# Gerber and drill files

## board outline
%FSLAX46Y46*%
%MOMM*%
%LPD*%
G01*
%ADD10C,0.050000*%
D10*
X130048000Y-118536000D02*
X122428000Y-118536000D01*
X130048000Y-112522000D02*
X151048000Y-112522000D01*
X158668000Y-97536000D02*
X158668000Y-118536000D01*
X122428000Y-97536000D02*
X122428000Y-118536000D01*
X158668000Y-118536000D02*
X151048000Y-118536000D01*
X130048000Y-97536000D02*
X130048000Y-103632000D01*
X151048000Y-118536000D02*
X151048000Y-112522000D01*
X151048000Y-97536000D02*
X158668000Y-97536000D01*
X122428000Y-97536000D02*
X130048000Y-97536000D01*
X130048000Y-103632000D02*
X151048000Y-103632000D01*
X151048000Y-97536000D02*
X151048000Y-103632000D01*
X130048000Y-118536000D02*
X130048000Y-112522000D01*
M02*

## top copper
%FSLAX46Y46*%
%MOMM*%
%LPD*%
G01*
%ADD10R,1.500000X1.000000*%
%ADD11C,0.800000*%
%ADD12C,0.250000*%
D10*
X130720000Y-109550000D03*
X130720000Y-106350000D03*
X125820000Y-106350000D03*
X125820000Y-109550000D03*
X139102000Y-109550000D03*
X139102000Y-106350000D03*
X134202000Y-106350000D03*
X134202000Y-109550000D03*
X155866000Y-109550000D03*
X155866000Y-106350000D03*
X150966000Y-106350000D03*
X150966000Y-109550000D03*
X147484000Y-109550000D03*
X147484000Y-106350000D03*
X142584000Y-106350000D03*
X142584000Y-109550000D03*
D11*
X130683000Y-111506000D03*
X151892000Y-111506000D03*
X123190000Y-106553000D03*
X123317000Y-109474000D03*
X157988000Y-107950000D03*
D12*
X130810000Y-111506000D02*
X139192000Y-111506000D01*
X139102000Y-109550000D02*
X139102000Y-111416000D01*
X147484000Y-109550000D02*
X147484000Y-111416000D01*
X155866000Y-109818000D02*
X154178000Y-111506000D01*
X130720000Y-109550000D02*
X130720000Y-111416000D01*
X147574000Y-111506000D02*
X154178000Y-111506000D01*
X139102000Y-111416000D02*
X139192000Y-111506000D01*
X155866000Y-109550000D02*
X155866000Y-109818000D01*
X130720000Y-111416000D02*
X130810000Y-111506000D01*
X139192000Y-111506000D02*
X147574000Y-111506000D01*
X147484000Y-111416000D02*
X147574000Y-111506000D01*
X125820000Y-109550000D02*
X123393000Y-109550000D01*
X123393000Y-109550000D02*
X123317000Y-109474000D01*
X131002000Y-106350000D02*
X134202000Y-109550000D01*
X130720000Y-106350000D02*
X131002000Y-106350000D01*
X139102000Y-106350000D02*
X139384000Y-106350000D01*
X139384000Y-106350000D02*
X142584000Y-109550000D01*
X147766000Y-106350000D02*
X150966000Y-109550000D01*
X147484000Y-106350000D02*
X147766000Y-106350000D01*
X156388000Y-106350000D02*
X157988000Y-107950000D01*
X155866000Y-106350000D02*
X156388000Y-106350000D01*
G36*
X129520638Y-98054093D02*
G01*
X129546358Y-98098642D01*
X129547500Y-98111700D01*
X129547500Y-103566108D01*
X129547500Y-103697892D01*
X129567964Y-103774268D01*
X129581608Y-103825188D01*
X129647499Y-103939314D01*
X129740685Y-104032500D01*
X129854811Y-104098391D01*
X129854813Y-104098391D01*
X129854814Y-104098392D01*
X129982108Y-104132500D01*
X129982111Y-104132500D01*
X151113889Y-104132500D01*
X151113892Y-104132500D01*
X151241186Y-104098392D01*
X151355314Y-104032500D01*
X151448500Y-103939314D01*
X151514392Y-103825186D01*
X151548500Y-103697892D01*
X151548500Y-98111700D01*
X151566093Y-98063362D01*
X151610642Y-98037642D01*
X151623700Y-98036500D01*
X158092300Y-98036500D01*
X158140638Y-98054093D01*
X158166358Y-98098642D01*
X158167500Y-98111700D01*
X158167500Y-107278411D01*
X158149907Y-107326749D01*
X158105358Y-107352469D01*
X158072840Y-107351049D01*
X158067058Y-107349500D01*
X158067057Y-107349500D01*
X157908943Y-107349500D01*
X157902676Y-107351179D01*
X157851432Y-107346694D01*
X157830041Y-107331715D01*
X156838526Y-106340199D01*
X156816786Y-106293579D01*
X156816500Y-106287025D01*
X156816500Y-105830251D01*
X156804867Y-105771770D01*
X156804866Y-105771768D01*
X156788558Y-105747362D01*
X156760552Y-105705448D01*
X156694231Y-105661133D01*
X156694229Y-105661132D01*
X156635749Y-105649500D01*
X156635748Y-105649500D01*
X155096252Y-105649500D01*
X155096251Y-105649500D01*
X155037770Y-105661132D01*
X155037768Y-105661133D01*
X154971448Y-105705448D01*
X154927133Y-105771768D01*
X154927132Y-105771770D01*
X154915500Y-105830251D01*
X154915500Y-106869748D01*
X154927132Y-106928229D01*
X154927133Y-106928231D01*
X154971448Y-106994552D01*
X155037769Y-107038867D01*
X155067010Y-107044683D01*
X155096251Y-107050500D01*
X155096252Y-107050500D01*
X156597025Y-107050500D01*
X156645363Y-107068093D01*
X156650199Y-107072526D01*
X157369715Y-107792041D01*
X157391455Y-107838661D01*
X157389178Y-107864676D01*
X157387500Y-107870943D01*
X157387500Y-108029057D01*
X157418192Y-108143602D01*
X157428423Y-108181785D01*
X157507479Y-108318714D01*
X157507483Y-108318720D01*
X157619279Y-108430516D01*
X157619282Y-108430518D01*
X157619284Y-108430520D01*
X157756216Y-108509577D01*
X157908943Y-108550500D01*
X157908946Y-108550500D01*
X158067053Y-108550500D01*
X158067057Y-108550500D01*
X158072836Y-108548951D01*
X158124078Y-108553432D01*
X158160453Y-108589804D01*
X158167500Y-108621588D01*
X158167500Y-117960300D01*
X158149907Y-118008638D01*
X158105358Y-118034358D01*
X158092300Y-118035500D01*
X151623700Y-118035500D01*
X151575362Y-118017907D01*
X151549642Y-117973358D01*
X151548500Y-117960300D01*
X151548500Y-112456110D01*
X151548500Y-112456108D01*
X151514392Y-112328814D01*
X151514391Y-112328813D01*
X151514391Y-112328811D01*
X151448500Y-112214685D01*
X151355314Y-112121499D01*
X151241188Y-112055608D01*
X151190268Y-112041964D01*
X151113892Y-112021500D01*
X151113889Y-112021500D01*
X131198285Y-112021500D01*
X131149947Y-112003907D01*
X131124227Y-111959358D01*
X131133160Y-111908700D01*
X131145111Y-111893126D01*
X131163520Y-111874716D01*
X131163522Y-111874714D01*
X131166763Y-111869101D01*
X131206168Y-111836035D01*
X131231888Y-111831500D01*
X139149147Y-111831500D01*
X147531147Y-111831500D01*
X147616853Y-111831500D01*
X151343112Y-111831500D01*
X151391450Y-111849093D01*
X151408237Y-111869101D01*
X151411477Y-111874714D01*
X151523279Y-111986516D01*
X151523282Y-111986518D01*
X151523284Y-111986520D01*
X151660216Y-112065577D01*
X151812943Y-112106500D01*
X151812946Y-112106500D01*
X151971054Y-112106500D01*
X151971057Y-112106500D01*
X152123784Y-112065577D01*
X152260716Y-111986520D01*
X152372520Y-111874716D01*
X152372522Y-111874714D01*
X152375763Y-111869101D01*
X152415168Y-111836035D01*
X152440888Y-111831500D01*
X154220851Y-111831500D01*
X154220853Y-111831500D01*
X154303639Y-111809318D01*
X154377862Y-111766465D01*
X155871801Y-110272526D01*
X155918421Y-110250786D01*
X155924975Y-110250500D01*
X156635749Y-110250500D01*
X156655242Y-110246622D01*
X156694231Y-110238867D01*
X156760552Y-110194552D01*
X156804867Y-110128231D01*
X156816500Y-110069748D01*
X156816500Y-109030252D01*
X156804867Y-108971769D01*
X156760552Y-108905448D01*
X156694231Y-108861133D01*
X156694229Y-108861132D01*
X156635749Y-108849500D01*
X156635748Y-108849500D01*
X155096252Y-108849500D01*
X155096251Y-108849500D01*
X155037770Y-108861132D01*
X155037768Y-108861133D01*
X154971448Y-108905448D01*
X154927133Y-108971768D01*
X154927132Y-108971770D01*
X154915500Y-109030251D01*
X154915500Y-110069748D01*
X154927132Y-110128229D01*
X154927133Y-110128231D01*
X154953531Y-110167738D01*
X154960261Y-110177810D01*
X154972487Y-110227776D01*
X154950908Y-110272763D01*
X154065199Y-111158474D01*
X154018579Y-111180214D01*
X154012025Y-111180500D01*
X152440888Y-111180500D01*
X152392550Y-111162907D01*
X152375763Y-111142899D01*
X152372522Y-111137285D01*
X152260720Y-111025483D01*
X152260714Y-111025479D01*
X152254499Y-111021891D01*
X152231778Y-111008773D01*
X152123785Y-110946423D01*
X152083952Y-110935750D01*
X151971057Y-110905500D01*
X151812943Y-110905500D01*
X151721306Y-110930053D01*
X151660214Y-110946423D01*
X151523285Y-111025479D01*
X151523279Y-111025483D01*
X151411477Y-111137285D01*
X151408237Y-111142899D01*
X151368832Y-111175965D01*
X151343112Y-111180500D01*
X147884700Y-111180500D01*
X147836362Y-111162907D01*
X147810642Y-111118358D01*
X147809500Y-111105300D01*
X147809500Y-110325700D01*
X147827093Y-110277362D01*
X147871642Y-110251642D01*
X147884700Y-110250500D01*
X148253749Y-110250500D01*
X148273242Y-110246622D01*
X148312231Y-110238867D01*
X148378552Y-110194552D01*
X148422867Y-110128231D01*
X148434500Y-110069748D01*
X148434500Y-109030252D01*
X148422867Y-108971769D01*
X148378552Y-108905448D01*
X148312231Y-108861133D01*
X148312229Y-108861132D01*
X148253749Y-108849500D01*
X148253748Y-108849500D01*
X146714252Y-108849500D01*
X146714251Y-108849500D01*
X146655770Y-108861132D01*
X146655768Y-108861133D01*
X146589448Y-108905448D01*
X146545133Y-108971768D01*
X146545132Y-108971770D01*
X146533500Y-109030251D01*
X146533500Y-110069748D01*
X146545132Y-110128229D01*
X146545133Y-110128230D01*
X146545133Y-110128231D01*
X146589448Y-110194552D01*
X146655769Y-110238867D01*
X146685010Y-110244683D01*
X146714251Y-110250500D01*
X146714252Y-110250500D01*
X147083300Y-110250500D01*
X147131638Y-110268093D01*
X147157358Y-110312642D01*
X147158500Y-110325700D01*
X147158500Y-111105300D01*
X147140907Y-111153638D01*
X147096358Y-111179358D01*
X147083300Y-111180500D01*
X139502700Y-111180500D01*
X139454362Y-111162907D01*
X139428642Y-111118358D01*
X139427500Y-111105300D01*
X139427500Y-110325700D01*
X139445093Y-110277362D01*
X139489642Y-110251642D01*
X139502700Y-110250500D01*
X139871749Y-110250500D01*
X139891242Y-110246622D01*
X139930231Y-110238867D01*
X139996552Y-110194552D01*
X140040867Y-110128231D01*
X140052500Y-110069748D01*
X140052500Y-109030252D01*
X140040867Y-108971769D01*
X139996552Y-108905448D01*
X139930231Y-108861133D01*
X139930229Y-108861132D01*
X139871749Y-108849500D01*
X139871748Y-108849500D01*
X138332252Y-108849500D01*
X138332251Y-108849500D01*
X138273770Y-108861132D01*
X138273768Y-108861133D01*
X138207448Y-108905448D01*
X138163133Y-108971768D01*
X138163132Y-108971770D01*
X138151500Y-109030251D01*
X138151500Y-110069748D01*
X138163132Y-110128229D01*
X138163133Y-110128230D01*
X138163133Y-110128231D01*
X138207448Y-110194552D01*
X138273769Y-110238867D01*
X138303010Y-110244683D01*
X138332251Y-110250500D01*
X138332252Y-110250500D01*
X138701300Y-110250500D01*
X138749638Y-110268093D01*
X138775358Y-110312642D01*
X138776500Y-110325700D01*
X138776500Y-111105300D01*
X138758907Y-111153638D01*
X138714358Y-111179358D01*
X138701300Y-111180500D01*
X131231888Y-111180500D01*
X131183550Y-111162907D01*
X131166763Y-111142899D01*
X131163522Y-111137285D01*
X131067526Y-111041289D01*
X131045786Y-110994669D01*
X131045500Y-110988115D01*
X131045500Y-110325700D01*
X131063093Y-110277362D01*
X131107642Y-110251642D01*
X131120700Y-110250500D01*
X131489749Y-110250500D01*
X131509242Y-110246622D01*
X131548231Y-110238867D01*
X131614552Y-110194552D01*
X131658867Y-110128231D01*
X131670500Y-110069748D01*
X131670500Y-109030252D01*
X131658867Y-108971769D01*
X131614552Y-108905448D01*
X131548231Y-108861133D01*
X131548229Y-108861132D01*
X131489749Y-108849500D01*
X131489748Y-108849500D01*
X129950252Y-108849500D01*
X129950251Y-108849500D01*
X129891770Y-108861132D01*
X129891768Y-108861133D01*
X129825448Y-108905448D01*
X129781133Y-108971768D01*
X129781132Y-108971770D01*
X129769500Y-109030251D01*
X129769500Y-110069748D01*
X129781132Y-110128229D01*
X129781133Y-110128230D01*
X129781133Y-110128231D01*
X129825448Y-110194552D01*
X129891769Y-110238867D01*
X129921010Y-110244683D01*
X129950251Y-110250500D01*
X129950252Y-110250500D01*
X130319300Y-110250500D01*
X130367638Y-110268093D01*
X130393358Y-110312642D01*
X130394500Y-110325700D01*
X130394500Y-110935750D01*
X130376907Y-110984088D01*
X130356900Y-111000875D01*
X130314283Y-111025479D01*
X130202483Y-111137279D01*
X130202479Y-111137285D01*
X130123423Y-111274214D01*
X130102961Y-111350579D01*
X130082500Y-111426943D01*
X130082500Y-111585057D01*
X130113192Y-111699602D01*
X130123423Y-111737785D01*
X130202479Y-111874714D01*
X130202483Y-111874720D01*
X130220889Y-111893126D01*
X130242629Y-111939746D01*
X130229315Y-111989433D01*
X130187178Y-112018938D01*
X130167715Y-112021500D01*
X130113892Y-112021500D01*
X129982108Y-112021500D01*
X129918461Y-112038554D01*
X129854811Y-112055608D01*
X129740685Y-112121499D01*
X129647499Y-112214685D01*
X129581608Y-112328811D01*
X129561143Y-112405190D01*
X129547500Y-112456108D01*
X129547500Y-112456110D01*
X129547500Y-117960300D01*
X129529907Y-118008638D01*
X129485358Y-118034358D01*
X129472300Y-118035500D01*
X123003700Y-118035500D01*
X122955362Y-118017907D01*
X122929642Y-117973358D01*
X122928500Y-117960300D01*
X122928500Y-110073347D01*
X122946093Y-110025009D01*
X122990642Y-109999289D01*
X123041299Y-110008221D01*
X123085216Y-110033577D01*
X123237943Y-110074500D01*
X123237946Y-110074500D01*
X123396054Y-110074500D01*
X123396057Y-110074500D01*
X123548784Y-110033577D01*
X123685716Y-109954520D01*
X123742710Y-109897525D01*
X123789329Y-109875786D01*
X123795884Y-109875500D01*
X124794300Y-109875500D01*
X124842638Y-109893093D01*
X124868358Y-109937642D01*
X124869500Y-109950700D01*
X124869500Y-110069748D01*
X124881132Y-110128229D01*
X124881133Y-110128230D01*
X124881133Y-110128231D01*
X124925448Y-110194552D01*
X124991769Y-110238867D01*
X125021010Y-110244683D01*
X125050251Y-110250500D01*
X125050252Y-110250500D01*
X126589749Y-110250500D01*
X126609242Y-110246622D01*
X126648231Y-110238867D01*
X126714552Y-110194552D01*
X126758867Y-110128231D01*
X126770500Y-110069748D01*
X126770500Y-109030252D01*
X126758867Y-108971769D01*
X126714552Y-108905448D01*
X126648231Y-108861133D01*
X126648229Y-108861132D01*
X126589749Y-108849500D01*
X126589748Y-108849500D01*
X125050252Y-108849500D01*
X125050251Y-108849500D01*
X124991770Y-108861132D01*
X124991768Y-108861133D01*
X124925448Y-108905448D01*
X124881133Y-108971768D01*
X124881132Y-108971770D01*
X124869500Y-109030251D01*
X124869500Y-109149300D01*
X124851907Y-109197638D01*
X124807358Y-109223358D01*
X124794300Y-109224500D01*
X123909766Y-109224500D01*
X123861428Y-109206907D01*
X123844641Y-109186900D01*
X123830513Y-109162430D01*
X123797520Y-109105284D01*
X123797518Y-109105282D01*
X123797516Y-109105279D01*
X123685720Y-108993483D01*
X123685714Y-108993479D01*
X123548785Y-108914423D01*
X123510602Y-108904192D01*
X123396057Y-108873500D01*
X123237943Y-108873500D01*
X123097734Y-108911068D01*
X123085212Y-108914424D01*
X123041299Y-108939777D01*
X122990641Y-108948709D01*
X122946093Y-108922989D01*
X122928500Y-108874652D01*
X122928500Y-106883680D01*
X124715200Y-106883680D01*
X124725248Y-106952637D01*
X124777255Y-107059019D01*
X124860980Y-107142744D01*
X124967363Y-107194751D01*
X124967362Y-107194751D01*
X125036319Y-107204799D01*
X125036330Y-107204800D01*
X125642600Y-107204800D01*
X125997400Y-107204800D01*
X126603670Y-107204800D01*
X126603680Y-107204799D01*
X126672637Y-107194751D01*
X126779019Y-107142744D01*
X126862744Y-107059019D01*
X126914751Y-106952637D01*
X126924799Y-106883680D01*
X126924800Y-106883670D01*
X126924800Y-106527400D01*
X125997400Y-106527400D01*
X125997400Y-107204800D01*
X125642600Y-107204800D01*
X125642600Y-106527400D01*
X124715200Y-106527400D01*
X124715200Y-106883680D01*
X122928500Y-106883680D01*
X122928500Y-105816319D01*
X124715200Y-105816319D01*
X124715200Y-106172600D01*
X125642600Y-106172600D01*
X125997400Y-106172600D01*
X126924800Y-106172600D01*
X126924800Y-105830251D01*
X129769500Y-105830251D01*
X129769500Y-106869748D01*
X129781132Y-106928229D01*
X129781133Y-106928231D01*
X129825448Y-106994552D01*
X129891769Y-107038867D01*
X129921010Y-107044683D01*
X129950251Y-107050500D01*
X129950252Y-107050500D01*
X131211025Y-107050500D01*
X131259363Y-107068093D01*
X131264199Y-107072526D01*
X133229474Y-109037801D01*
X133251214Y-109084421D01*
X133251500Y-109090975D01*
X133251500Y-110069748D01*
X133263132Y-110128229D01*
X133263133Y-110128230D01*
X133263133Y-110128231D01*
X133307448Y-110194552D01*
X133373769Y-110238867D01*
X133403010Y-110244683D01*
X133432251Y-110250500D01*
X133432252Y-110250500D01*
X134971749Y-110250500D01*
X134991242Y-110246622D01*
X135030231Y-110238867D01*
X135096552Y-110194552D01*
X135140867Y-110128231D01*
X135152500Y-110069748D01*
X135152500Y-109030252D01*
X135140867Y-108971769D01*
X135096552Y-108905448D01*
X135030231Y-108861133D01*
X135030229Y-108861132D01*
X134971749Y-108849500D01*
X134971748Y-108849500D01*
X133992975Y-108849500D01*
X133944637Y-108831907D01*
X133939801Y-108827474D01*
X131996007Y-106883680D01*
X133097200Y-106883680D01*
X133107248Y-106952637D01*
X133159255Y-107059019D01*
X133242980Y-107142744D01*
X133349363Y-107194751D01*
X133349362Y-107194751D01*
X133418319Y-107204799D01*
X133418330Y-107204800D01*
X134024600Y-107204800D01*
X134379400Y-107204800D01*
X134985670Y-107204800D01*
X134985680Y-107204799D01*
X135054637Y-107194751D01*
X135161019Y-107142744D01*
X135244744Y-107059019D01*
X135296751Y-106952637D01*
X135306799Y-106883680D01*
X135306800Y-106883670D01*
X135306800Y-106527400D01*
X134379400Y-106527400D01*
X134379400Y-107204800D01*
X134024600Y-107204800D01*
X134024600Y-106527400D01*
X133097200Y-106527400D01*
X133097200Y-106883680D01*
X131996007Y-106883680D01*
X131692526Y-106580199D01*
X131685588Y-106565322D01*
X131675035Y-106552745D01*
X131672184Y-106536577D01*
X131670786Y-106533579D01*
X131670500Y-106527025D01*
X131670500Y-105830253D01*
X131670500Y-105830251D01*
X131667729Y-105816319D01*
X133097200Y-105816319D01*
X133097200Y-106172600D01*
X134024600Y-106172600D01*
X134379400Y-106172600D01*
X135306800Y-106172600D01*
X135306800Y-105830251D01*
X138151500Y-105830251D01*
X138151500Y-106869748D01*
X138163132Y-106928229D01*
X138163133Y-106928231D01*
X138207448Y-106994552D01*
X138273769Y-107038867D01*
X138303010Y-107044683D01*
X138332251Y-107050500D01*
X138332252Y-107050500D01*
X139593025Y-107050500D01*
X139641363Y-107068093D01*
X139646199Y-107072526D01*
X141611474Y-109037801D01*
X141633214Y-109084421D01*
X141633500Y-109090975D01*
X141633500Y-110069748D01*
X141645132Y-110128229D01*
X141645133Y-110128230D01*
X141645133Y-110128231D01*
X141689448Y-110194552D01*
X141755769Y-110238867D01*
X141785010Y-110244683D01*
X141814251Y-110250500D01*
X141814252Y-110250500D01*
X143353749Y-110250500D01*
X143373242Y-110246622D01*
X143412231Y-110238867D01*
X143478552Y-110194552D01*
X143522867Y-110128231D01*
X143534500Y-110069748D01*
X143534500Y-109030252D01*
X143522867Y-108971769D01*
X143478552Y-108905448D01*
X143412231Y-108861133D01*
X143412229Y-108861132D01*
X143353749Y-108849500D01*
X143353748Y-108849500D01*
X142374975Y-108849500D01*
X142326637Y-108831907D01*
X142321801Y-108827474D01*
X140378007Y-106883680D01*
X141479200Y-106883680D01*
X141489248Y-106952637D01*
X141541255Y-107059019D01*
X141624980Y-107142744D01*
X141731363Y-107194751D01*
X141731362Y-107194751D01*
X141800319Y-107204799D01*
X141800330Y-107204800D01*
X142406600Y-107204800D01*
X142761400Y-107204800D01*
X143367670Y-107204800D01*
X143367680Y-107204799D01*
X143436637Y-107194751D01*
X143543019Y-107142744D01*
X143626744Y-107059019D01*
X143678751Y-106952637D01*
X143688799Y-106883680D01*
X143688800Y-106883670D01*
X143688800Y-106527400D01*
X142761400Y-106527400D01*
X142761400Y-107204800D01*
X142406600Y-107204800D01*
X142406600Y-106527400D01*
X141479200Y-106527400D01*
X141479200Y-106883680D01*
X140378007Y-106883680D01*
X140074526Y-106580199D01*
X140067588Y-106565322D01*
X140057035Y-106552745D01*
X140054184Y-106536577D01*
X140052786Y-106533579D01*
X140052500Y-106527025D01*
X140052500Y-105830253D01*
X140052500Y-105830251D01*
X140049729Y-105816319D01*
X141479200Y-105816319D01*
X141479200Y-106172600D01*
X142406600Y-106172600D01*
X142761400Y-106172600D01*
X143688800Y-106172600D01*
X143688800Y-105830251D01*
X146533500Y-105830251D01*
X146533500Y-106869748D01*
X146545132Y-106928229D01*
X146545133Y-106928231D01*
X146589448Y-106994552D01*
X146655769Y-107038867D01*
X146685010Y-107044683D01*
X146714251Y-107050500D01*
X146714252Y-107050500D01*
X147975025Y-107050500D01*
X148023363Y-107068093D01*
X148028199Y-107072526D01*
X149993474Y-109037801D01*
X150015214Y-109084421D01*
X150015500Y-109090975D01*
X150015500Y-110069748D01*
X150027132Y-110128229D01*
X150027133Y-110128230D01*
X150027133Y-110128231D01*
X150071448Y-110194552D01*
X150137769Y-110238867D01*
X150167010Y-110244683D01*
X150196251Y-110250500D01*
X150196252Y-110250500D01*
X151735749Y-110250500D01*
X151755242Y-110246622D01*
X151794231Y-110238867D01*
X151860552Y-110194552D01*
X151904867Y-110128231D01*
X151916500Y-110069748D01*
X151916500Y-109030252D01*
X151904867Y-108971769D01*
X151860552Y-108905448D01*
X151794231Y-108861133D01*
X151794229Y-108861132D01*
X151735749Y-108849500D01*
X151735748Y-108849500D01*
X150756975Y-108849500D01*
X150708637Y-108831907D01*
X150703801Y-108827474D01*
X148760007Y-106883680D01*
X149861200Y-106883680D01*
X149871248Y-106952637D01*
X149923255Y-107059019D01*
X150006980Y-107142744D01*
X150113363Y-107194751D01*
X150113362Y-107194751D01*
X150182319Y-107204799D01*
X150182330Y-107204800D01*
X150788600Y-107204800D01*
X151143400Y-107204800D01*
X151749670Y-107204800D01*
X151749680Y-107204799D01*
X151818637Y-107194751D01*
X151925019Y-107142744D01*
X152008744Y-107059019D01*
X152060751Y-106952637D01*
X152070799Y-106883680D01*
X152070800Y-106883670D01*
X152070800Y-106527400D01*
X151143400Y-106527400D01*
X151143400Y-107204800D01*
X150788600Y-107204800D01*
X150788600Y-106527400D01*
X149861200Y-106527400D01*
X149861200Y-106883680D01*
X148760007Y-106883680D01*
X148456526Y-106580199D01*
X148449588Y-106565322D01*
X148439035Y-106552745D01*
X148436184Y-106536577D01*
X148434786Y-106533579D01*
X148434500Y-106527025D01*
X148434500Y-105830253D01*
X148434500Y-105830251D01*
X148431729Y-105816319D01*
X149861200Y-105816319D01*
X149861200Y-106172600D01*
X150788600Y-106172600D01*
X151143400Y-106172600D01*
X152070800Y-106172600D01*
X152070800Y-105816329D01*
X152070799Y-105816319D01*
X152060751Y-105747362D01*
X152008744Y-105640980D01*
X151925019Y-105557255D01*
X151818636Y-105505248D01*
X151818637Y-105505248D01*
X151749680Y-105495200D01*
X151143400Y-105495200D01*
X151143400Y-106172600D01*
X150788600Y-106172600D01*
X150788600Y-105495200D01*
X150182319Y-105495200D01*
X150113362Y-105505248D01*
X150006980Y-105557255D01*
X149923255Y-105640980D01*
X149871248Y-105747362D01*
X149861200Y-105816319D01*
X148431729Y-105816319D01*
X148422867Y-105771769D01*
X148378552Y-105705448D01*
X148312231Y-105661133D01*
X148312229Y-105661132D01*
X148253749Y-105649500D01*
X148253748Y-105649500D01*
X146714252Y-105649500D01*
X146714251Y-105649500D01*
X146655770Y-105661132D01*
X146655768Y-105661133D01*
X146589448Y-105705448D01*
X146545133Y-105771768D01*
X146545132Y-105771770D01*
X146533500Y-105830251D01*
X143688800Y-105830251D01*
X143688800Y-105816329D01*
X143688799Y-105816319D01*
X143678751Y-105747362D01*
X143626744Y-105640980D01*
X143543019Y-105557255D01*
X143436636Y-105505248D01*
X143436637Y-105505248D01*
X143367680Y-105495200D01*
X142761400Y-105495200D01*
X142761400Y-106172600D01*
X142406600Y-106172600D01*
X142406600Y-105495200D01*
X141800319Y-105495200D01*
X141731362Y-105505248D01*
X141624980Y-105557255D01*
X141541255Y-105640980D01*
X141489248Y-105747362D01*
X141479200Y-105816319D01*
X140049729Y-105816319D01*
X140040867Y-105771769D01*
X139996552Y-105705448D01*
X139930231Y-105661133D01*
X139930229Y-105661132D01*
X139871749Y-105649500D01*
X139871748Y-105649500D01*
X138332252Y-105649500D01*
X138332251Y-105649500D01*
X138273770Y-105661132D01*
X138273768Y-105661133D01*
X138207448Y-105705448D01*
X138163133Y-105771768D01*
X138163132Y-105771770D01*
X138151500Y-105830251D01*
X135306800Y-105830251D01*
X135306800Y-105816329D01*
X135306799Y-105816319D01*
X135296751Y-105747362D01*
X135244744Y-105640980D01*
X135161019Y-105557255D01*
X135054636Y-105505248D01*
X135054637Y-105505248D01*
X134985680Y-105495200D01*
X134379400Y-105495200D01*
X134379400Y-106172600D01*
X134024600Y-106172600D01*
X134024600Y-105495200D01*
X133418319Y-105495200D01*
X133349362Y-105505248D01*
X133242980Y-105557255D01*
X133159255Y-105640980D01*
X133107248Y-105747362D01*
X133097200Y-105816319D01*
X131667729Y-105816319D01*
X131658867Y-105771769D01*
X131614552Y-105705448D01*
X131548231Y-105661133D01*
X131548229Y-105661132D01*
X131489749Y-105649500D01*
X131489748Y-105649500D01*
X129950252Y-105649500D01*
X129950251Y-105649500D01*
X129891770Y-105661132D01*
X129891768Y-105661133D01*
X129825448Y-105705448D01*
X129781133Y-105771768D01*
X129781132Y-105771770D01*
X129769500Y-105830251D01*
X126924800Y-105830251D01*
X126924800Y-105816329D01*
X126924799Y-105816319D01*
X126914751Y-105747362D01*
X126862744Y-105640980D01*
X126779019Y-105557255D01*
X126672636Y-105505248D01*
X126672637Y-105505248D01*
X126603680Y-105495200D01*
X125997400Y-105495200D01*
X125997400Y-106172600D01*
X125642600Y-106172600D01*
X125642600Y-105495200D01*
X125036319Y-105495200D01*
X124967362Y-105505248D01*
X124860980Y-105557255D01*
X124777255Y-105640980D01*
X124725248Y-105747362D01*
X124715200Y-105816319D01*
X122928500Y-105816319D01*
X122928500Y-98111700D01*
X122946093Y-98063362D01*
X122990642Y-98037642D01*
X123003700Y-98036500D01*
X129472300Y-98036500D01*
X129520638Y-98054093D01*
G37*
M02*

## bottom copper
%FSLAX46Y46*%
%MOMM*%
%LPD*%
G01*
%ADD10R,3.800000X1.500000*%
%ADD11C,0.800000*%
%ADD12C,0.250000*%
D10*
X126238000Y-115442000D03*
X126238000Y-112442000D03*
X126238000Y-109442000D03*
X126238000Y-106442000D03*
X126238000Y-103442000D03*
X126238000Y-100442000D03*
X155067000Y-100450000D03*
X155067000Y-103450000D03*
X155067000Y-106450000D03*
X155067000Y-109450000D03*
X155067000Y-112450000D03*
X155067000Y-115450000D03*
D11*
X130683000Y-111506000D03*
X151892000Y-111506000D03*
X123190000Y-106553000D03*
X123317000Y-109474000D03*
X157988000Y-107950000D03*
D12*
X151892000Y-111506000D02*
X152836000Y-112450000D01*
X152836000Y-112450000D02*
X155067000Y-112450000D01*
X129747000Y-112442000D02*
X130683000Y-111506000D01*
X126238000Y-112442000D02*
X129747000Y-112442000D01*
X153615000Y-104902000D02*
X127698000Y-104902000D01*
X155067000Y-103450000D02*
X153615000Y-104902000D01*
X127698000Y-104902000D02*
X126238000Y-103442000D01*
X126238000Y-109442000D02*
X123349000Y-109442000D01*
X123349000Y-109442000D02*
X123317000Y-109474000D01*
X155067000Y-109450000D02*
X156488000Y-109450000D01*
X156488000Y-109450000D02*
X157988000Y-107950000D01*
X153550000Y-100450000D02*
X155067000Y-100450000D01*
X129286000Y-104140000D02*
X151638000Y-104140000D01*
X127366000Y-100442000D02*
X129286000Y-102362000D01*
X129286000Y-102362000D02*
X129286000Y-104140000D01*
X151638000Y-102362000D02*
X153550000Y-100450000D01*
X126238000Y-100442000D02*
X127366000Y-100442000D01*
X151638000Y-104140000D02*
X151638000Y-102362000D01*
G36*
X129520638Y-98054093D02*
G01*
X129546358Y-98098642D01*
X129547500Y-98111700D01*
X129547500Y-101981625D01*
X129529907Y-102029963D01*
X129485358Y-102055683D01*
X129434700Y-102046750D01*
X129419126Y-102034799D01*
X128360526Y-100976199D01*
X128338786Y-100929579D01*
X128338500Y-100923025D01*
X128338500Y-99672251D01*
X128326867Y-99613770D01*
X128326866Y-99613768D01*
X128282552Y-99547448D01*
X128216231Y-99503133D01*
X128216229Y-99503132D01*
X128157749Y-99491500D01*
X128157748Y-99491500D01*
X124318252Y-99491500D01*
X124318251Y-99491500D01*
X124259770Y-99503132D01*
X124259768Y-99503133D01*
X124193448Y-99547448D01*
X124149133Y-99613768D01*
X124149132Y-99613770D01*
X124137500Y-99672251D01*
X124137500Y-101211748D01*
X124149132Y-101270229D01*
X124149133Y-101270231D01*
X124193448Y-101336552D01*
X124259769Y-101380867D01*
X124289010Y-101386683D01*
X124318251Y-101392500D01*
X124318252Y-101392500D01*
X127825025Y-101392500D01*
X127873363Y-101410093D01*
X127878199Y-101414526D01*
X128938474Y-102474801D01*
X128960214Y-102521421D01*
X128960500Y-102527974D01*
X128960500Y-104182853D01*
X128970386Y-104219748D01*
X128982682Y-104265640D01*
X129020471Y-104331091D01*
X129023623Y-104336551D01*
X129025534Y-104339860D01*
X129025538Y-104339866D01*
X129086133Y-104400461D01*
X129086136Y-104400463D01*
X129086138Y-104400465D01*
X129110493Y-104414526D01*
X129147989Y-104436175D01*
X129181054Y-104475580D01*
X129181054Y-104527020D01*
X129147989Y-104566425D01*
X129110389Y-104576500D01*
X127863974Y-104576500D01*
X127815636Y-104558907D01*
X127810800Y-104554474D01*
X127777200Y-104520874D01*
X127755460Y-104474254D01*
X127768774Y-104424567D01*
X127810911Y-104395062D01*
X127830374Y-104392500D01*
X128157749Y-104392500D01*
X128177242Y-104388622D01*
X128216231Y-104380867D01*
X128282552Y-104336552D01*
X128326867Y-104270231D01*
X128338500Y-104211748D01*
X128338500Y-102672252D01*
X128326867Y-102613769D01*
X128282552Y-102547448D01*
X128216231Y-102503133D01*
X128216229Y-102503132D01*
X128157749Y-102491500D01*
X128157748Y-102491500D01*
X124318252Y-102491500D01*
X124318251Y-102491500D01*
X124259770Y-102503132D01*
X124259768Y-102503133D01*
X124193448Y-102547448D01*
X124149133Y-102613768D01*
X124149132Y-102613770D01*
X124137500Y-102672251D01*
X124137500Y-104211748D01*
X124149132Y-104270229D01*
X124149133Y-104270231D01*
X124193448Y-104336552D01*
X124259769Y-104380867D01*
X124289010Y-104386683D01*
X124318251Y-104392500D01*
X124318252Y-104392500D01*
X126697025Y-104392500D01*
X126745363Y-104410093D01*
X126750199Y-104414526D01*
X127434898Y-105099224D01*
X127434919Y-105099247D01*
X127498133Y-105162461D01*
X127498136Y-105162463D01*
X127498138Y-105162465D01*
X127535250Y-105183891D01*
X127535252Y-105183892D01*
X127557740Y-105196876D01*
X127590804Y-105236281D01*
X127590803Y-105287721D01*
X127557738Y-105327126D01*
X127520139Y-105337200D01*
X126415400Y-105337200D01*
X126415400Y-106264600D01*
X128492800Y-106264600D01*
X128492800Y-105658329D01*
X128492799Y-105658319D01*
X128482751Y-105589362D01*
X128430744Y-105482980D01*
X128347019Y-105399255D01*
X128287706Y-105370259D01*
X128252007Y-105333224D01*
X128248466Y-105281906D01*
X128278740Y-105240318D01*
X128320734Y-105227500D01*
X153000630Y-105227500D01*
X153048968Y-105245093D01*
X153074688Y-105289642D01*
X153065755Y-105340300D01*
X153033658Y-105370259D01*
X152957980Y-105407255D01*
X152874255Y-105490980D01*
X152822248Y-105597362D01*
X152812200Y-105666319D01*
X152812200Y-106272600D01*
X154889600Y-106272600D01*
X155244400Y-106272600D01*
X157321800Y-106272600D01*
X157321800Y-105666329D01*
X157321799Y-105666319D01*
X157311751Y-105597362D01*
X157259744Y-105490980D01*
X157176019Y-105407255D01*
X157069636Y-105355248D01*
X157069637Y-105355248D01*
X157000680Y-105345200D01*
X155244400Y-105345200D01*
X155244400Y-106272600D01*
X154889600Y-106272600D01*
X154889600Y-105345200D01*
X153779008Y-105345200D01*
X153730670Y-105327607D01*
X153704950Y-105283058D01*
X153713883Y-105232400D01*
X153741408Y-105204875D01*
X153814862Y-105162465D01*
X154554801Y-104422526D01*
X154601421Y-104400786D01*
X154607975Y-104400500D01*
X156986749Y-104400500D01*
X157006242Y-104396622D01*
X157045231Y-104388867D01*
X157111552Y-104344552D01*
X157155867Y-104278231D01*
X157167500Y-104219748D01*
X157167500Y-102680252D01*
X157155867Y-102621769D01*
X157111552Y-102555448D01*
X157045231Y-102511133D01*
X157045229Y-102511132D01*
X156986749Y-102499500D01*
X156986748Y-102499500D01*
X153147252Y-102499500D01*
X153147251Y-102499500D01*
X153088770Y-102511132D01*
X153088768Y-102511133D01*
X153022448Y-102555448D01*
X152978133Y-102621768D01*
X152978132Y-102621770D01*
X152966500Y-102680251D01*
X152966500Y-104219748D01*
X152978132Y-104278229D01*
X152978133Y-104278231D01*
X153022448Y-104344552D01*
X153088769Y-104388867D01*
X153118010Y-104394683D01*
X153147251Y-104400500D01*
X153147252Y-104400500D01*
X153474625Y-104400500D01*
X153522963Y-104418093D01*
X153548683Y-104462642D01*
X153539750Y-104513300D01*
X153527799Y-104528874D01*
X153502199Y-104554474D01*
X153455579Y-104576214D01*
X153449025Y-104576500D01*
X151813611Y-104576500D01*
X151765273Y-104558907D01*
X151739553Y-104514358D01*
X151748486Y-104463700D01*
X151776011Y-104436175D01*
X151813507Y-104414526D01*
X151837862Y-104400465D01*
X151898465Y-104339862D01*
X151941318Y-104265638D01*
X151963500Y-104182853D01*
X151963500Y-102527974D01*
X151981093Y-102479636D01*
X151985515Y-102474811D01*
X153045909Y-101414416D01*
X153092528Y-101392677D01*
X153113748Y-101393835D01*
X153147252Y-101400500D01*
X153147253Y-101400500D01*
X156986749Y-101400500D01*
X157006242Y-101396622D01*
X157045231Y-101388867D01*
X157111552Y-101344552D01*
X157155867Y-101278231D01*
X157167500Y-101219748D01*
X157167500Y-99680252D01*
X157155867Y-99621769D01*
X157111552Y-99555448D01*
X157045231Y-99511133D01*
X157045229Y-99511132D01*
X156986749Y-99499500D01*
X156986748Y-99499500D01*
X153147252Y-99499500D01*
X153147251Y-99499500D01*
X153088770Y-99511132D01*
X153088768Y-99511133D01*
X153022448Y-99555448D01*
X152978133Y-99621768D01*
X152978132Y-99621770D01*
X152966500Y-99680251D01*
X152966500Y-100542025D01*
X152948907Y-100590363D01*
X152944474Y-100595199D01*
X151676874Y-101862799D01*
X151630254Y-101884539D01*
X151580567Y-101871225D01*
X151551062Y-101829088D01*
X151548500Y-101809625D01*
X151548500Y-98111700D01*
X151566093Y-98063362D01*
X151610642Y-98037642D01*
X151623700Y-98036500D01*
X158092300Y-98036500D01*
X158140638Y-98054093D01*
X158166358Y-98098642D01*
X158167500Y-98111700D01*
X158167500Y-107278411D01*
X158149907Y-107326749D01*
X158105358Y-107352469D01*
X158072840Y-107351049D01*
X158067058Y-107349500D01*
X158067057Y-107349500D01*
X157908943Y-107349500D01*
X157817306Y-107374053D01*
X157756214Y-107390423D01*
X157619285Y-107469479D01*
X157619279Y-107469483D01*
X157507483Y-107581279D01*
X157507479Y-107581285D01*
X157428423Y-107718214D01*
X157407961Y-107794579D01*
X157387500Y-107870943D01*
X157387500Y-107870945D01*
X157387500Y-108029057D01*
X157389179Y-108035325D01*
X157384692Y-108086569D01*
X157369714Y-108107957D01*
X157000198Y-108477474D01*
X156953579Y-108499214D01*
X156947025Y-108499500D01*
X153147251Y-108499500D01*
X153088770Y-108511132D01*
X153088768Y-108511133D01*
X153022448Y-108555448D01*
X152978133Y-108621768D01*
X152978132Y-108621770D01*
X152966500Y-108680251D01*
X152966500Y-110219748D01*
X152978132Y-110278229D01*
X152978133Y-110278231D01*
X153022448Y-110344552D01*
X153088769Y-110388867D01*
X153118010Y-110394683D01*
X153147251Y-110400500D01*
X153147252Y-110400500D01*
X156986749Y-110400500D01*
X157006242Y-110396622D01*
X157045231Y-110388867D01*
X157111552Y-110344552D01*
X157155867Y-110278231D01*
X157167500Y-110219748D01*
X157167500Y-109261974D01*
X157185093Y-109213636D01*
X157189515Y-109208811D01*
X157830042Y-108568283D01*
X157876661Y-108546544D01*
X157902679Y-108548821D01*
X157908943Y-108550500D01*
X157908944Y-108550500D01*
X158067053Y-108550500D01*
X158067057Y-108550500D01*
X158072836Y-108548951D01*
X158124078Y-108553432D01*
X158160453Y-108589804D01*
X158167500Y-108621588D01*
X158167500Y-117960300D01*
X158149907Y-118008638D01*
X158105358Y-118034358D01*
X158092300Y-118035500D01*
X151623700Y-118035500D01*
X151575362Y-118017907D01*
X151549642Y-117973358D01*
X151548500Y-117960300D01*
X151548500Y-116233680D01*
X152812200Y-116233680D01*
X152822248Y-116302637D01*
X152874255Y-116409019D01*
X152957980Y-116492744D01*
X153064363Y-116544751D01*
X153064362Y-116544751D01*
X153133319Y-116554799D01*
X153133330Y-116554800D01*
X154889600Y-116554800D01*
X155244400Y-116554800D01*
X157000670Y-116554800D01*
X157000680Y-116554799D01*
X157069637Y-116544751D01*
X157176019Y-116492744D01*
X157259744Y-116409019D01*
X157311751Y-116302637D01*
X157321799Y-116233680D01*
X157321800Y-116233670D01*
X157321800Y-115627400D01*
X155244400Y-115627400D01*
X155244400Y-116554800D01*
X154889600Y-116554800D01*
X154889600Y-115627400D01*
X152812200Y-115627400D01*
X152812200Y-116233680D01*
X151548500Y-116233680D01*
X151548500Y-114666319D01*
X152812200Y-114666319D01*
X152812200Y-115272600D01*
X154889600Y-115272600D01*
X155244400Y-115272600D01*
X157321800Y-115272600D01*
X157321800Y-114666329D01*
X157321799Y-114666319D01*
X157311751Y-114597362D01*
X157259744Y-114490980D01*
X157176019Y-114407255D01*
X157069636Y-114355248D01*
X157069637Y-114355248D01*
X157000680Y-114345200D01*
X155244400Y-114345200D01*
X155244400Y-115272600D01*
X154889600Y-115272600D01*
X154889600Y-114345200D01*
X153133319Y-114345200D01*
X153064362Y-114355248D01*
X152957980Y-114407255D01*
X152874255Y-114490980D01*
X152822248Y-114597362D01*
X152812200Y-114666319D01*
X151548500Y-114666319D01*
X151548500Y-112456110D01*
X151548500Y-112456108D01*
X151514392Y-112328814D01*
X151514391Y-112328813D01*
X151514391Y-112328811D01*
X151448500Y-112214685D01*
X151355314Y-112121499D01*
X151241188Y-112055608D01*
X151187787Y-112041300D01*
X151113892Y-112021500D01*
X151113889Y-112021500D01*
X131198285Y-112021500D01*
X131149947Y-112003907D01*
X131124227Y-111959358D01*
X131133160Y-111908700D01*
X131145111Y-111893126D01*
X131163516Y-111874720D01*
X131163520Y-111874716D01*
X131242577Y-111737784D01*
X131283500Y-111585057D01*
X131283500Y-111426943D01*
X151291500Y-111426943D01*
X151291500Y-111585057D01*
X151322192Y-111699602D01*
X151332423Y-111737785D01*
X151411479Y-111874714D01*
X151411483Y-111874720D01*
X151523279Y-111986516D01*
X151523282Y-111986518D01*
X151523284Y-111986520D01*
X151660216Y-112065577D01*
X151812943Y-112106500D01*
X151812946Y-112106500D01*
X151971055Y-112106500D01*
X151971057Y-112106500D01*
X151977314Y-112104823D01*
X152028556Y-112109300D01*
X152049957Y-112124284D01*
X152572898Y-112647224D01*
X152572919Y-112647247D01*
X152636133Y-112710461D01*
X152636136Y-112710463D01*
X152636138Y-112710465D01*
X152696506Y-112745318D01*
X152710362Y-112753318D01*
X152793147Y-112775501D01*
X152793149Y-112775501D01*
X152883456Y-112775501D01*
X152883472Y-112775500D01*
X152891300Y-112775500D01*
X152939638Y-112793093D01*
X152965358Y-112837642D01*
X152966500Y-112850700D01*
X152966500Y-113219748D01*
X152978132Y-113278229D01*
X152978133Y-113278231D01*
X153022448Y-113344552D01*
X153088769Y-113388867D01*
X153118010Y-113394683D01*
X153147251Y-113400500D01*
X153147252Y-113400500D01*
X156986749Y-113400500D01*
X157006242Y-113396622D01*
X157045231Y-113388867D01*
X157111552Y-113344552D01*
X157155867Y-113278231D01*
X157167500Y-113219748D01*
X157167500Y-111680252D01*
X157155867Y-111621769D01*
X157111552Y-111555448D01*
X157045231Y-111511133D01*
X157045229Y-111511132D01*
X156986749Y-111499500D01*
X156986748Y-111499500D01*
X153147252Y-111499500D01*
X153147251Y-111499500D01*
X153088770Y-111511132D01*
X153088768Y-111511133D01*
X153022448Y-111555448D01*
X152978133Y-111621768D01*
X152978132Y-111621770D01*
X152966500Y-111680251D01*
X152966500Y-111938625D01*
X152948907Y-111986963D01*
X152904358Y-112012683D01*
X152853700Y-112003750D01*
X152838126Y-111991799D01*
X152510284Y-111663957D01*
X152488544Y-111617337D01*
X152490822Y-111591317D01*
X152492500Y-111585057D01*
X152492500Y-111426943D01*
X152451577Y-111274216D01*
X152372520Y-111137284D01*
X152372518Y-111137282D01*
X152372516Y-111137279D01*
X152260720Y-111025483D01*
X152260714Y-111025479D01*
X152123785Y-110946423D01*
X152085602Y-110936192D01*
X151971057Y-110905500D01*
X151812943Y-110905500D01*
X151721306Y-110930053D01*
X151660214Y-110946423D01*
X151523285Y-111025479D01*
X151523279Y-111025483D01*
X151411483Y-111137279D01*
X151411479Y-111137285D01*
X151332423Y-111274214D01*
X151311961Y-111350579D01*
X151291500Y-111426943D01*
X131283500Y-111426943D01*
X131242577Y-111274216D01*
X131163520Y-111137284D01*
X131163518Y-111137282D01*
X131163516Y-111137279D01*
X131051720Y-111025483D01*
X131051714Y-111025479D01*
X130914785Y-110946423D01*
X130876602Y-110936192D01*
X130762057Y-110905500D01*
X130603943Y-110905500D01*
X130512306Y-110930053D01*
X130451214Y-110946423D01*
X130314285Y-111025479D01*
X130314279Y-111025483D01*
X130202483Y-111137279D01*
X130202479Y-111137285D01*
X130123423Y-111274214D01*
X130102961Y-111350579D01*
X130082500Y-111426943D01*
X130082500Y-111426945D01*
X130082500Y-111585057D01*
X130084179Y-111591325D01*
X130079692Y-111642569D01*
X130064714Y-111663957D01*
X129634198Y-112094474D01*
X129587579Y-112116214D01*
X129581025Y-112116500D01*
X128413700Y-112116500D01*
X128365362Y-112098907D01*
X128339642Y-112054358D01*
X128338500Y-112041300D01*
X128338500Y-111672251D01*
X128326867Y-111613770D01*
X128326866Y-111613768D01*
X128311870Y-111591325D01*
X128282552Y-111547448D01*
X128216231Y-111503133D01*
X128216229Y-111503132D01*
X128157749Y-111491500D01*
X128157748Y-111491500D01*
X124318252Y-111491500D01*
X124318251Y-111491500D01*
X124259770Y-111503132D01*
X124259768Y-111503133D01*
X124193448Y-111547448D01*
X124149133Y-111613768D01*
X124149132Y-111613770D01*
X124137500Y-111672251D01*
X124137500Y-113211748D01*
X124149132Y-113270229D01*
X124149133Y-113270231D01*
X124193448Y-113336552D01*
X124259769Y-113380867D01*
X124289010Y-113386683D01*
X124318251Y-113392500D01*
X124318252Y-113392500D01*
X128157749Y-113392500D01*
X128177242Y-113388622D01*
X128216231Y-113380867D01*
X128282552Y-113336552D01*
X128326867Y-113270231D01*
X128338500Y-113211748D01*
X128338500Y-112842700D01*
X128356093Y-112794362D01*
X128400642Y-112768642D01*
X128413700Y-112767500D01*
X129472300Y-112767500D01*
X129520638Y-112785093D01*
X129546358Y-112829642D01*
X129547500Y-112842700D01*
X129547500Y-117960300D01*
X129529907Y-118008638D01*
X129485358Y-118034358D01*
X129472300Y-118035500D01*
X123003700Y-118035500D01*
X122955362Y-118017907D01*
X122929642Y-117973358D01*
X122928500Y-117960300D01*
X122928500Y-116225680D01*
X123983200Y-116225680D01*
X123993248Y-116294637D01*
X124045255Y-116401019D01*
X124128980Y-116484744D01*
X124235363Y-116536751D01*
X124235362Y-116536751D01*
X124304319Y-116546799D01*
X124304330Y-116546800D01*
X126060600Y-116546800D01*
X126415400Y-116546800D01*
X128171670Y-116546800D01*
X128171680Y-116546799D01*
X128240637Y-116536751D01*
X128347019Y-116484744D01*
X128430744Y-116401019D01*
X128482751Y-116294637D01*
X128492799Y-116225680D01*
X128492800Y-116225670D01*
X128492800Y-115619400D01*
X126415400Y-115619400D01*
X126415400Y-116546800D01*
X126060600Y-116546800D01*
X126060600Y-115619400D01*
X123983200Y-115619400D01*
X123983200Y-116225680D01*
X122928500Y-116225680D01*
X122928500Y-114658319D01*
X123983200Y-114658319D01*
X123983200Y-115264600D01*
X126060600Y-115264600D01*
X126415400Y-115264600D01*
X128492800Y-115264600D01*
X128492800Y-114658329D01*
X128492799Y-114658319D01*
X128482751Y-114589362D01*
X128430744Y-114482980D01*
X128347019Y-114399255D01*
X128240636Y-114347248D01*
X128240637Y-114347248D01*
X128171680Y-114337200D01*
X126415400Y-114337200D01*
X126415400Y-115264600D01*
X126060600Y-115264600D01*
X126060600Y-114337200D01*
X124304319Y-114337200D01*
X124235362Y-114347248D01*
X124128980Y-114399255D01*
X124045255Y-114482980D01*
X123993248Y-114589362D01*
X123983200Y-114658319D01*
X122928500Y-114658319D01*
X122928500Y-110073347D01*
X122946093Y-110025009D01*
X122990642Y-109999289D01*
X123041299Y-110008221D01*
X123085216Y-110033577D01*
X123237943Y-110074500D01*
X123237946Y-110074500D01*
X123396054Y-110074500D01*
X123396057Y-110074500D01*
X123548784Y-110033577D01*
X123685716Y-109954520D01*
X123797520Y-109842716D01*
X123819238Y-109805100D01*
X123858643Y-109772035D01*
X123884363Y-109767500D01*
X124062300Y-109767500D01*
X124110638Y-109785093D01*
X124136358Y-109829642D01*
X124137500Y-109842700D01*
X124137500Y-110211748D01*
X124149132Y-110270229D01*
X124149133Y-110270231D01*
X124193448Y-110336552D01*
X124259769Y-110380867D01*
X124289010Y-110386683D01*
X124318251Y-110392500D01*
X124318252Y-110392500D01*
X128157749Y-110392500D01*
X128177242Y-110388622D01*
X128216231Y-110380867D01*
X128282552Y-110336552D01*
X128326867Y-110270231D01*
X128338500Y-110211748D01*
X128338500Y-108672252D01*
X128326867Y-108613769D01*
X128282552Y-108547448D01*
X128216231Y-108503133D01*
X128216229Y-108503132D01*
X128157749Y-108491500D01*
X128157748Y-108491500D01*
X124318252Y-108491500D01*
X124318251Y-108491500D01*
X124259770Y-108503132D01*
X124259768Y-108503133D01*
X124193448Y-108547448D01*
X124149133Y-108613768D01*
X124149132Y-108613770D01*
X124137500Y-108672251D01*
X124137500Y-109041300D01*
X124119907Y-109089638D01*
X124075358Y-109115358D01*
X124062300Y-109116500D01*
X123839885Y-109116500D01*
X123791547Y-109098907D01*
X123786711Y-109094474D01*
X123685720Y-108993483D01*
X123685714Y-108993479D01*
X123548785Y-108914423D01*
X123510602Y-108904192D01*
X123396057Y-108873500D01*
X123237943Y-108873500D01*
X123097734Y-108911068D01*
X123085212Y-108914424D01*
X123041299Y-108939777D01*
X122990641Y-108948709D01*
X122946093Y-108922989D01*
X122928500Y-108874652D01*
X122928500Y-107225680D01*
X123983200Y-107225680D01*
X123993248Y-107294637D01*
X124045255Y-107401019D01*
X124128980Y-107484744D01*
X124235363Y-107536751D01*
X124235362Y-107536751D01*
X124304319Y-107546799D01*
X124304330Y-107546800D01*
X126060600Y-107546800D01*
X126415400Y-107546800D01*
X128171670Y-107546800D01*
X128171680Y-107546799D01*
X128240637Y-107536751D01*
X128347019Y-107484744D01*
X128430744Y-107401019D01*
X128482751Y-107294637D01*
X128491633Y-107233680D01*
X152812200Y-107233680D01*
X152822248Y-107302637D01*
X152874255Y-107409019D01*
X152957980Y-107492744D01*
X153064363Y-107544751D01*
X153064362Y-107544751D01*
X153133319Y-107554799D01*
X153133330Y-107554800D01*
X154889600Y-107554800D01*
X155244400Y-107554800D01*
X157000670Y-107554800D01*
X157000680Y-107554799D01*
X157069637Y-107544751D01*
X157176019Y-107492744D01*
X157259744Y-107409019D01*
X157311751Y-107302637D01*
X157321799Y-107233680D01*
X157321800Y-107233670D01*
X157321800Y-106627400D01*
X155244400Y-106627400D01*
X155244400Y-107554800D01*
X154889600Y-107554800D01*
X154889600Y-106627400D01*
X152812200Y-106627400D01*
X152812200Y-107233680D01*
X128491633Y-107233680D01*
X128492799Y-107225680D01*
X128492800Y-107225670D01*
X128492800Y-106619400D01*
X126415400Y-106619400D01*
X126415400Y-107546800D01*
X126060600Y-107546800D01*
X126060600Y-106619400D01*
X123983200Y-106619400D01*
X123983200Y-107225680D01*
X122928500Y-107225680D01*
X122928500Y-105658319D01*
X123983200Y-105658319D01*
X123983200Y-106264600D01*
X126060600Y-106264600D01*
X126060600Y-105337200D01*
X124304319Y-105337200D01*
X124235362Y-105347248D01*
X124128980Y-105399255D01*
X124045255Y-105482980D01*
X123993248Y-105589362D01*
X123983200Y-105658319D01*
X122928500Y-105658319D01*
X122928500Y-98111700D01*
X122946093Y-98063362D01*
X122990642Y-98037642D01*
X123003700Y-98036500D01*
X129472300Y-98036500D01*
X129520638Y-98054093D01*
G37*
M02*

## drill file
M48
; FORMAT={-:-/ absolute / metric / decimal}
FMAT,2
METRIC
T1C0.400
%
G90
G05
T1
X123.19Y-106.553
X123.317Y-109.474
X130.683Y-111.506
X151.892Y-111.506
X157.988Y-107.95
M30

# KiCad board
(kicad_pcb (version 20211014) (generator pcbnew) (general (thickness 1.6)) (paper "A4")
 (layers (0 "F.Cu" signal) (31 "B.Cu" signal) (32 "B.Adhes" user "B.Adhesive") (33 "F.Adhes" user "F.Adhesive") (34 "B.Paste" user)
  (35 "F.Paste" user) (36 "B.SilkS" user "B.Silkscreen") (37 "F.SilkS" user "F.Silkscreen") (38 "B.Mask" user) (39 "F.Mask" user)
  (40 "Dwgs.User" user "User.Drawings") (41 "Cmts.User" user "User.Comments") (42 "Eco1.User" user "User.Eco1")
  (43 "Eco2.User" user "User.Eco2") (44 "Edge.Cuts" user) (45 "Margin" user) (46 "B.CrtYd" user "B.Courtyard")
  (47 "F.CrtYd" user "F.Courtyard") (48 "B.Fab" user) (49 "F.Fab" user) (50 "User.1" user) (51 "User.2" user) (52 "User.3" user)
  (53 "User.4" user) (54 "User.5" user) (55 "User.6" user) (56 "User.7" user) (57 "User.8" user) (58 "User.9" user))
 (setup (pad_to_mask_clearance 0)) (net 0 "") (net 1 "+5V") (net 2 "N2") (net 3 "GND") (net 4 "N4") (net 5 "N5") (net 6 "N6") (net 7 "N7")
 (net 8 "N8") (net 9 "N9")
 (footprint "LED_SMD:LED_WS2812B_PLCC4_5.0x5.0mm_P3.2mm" (layer "F.Cu") (at 128.27 107.95 180)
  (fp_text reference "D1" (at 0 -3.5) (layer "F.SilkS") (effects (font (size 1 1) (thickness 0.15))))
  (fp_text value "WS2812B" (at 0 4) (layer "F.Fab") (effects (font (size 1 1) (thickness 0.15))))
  (pad "1" smd rect (at -2.45 -1.6 180) (size 1.5 1) (layers "F.Cu" "F.Paste" "F.Mask") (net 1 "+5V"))
  (pad "2" smd rect (at -2.45 1.6 180) (size 1.5 1) (layers "F.Cu" "F.Paste" "F.Mask") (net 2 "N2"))
  (pad "3" smd rect (at 2.45 1.6 180) (size 1.5 1) (layers "F.Cu" "F.Paste" "F.Mask") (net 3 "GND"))
  (pad "4" smd rect (at 2.45 -1.6 180) (size 1.5 1) (layers "F.Cu" "F.Paste" "F.Mask") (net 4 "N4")))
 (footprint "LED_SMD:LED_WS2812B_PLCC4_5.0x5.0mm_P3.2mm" (layer "F.Cu") (at 136.652 107.95 180)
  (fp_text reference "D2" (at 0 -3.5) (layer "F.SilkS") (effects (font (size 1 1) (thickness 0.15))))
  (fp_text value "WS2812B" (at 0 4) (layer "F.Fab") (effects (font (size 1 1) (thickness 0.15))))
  (pad "1" smd rect (at -2.45 -1.6 180) (size 1.5 1) (layers "F.Cu" "F.Paste" "F.Mask") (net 1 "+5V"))
  (pad "2" smd rect (at -2.45 1.6 180) (size 1.5 1) (layers "F.Cu" "F.Paste" "F.Mask") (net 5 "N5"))
  (pad "3" smd rect (at 2.45 1.6 180) (size 1.5 1) (layers "F.Cu" "F.Paste" "F.Mask") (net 3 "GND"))
  (pad "4" smd rect (at 2.45 -1.6 180) (size 1.5 1) (layers "F.Cu" "F.Paste" "F.Mask") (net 2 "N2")))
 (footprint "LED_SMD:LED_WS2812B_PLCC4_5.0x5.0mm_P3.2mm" (layer "F.Cu") (at 153.416 107.95 180)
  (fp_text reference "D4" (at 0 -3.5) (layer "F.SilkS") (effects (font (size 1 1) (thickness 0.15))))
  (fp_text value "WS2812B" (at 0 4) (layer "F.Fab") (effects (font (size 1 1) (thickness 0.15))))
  (pad "1" smd rect (at -2.45 -1.6 180) (size 1.5 1) (layers "F.Cu" "F.Paste" "F.Mask") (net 1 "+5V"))
  (pad "2" smd rect (at -2.45 1.6 180) (size 1.5 1) (layers "F.Cu" "F.Paste" "F.Mask") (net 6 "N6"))
  (pad "3" smd rect (at 2.45 1.6 180) (size 1.5 1) (layers "F.Cu" "F.Paste" "F.Mask") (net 3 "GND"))
  (pad "4" smd rect (at 2.45 -1.6 180) (size 1.5 1) (layers "F.Cu" "F.Paste" "F.Mask") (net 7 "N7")))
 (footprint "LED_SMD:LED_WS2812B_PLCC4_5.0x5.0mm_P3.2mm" (layer "F.Cu") (at 145.034 107.95 180)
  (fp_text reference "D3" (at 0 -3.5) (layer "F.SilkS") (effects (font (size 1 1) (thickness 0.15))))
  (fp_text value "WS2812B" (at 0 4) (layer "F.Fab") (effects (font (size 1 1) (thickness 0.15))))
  (pad "1" smd rect (at -2.45 -1.6 180) (size 1.5 1) (layers "F.Cu" "F.Paste" "F.Mask") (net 1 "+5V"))
  (pad "2" smd rect (at -2.45 1.6 180) (size 1.5 1) (layers "F.Cu" "F.Paste" "F.Mask") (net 7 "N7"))
  (pad "3" smd rect (at 2.45 1.6 180) (size 1.5 1) (layers "F.Cu" "F.Paste" "F.Mask") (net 3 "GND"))
  (pad "4" smd rect (at 2.45 -1.6 180) (size 1.5 1) (layers "F.Cu" "F.Paste" "F.Mask") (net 5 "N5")))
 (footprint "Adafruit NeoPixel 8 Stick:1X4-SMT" (layer "B.Cu") (at 126.873 107.442 90)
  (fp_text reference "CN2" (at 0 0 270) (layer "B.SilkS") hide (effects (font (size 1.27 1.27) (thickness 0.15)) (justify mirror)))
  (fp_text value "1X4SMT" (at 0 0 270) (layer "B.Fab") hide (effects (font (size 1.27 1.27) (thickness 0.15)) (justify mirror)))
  (pad "1" smd rect (at -8 -0.635 90) (size 1.5 3.8) (layers "B.Cu" "B.Paste" "B.Mask") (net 3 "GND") (solder_mask_margin 0.1016))
  (pad "2" smd rect (at -5 -0.635 90) (size 1.5 3.8) (layers "B.Cu" "B.Paste" "B.Mask") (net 1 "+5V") (solder_mask_margin 0.1016))
  (pad "3" smd rect (at -2 -0.635 90) (size 1.5 3.8) (layers "B.Cu" "B.Paste" "B.Mask") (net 4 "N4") (solder_mask_margin 0.1016))
  (pad "4" smd rect (at 1 -0.635 90) (size 1.5 3.8) (layers "B.Cu" "B.Paste" "B.Mask") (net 3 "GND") (solder_mask_margin 0.1016))
  (pad "5" smd rect (at 4 -0.635 90) (size 1.5 3.8) (layers "B.Cu" "B.Paste" "B.Mask") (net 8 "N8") (solder_mask_margin 0.1016))
  (pad "6" smd rect (at 7 -0.635 90) (size 1.5 3.8) (layers "B.Cu" "B.Paste" "B.Mask") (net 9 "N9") (solder_mask_margin 0.1016)))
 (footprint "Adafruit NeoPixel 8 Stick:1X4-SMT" (layer "B.Cu") (at 154.432 108.45 -90)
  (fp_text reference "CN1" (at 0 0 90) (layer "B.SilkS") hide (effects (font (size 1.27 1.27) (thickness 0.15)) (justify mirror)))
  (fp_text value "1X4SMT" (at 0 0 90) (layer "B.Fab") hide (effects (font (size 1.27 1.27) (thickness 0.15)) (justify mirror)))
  (pad "1" smd rect (at -8 -0.635 270) (size 1.5 3.8) (layers "B.Cu" "B.Paste" "B.Mask") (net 9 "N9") (solder_mask_margin 0.1016))
  (pad "2" smd rect (at -5 -0.635 270) (size 1.5 3.8) (layers "B.Cu" "B.Paste" "B.Mask") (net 8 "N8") (solder_mask_margin 0.1016))
  (pad "3" smd rect (at -2 -0.635 270) (size 1.5 3.8) (layers "B.Cu" "B.Paste" "B.Mask") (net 3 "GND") (solder_mask_margin 0.1016))
  (pad "4" smd rect (at 1 -0.635 270) (size 1.5 3.8) (layers "B.Cu" "B.Paste" "B.Mask") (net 6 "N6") (solder_mask_margin 0.1016))
  (pad "5" smd rect (at 4 -0.635 270) (size 1.5 3.8) (layers "B.Cu" "B.Paste" "B.Mask") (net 1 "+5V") (solder_mask_margin 0.1016))
  (pad "6" smd rect (at 7 -0.635 270) (size 1.5 3.8) (layers "B.Cu" "B.Paste" "B.Mask") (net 3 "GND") (solder_mask_margin 0.1016)))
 (gr_line (start 130.048 118.536) (end 122.428 118.536) (layer "Edge.Cuts") (width 0.05))
 (gr_line (start 130.048 112.522) (end 151.048 112.522) (layer "Edge.Cuts") (width 0.05))
 (gr_line (start 158.668 97.536) (end 158.668 118.536) (layer "Edge.Cuts") (width 0.05))
 (gr_line (start 122.428 97.536) (end 122.428 118.536) (layer "Edge.Cuts") (width 0.05))
 (gr_line locked (start 158.668 118.536) (end 151.048 118.536) (layer "Edge.Cuts") (width 0.05))
 (gr_line (start 130.048 97.536) (end 130.048 103.632) (layer "Edge.Cuts") (width 0.05))
 (gr_line (start 151.048 118.536) (end 151.048 112.522) (layer "Edge.Cuts") (width 0.05))
 (gr_line (start 151.048 97.536) (end 158.668 97.536) (layer "Edge.Cuts") (width 0.05))
 (gr_line (start 122.428 97.536) (end 130.048 97.536) (layer "Edge.Cuts") (width 0.05))
 (gr_line (start 130.048 103.632) (end 151.048 103.632) (layer "Edge.Cuts") (width 0.05))
 (gr_line (start 151.048 97.536) (end 151.048 103.632) (layer "Edge.Cuts") (width 0.05))
 (gr_line (start 130.048 118.536) (end 130.048 112.522) (layer "Edge.Cuts") (width 0.05))
 (segment (start 130.81 111.506) (end 139.192 111.506) (width 0.25) (layer "F.Cu") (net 1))
 (segment (start 139.102 109.55) (end 139.102 111.416) (width 0.25) (layer "F.Cu") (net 1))
 (segment (start 147.484 109.55) (end 147.484 111.416) (width 0.25) (layer "F.Cu") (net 1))
 (segment (start 155.866 109.818) (end 154.178 111.506) (width 0.25) (layer "F.Cu") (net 1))
 (segment (start 130.72 109.55) (end 130.72 111.416) (width 0.25) (layer "F.Cu") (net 1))
 (segment (start 147.574 111.506) (end 154.178 111.506) (width 0.25) (layer "F.Cu") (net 1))
 (segment (start 139.102 111.416) (end 139.192 111.506) (width 0.25) (layer "F.Cu") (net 1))
 (segment (start 155.866 109.55) (end 155.866 109.818) (width 0.25) (layer "F.Cu") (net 1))
 (segment (start 130.72 111.416) (end 130.81 111.506) (width 0.25) (layer "F.Cu") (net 1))
 (segment (start 139.192 111.506) (end 147.574 111.506) (width 0.25) (layer "F.Cu") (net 1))
 (segment (start 147.484 111.416) (end 147.574 111.506) (width 0.25) (layer "F.Cu") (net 1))
 (via (at 130.683 111.506) (size 0.8) (drill 0.4) (layers "F.Cu" "B.Cu") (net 1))
 (via (at 151.892 111.506) (size 0.8) (drill 0.4) (layers "F.Cu" "B.Cu") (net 1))
 (segment (start 151.892 111.506) (end 152.836 112.45) (width 0.25) (layer "B.Cu") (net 1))
 (segment (start 152.836 112.45) (end 155.067 112.45) (width 0.25) (layer "B.Cu") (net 1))
 (segment (start 129.747 112.442) (end 130.683 111.506) (width 0.25) (layer "B.Cu") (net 1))
 (segment (start 126.238 112.442) (end 129.747 112.442) (width 0.25) (layer "B.Cu") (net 1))
 (via (at 123.19 106.553) (size 0.8) (drill 0.4) (layers "F.Cu" "B.Cu") (free) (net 3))
 (segment (start 153.615 104.902) (end 127.698 104.902) (width 0.25) (layer "B.Cu") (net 8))
 (segment (start 155.067 103.45) (end 153.615 104.902) (width 0.25) (layer "B.Cu") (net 8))
 (segment (start 127.698 104.902) (end 126.238 103.442) (width 0.25) (layer "B.Cu") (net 8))
 (segment (start 125.82 109.55) (end 123.393 109.55) (width 0.25) (layer "F.Cu") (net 4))
 (segment (start 123.393 109.55) (end 123.317 109.474) (width 0.25) (layer "F.Cu") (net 4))
 (via (at 123.317 109.474) (size 0.8) (drill 0.4) (layers "F.Cu" "B.Cu") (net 4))
 (segment (start 126.238 109.442) (end 123.349 109.442) (width 0.25) (layer "B.Cu") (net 4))
 (segment (start 123.349 109.442) (end 123.317 109.474) (width 0.25) (layer "B.Cu") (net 4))
 (segment (start 131.002 106.35) (end 134.202 109.55) (width 0.25) (layer "F.Cu") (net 2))
 (segment (start 130.72 106.35) (end 131.002 106.35) (width 0.25) (layer "F.Cu") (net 2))
 (segment (start 139.102 106.35) (end 139.384 106.35) (width 0.25) (layer "F.Cu") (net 5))
 (segment (start 139.384 106.35) (end 142.584 109.55) (width 0.25) (layer "F.Cu") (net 5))
 (segment (start 147.766 106.35) (end 150.966 109.55) (width 0.25) (layer "F.Cu") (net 7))
 (segment (start 147.484 106.35) (end 147.766 106.35) (width 0.25) (layer "F.Cu") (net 7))
 (segment (start 156.388 106.35) (end 157.988 107.95) (width 0.25) (layer "F.Cu") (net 6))
 (segment (start 155.866 106.35) (end 156.388 106.35) (width 0.25) (layer "F.Cu") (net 6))
 (via (at 157.988 107.95) (size 0.8) (drill 0.4) (layers "F.Cu" "B.Cu") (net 6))
 (segment (start 155.067 109.45) (end 156.488 109.45) (width 0.25) (layer "B.Cu") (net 6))
 (segment (start 156.488 109.45) (end 157.988 107.95) (width 0.25) (layer "B.Cu") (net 6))
 (segment (start 153.55 100.45) (end 155.067 100.45) (width 0.25) (layer "B.Cu") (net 9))
 (segment (start 129.286 104.14) (end 151.638 104.14) (width 0.25) (layer "B.Cu") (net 9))
 (segment (start 127.366 100.442) (end 129.286 102.362) (width 0.25) (layer "B.Cu") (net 9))
 (segment (start 129.286 102.362) (end 129.286 104.14) (width 0.25) (layer "B.Cu") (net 9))
 (segment (start 151.638 102.362) (end 153.55 100.45) (width 0.25) (layer "B.Cu") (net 9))
 (segment (start 126.238 100.442) (end 127.366 100.442) (width 0.25) (layer "B.Cu") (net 9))
 (segment (start 151.638 104.14) (end 151.638 102.362) (width 0.25) (layer "B.Cu") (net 9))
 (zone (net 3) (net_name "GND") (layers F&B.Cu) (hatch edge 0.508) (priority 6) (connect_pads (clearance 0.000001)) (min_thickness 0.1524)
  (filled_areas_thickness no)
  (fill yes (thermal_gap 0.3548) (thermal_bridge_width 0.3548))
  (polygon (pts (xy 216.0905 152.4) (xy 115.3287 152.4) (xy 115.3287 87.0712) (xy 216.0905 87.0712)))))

